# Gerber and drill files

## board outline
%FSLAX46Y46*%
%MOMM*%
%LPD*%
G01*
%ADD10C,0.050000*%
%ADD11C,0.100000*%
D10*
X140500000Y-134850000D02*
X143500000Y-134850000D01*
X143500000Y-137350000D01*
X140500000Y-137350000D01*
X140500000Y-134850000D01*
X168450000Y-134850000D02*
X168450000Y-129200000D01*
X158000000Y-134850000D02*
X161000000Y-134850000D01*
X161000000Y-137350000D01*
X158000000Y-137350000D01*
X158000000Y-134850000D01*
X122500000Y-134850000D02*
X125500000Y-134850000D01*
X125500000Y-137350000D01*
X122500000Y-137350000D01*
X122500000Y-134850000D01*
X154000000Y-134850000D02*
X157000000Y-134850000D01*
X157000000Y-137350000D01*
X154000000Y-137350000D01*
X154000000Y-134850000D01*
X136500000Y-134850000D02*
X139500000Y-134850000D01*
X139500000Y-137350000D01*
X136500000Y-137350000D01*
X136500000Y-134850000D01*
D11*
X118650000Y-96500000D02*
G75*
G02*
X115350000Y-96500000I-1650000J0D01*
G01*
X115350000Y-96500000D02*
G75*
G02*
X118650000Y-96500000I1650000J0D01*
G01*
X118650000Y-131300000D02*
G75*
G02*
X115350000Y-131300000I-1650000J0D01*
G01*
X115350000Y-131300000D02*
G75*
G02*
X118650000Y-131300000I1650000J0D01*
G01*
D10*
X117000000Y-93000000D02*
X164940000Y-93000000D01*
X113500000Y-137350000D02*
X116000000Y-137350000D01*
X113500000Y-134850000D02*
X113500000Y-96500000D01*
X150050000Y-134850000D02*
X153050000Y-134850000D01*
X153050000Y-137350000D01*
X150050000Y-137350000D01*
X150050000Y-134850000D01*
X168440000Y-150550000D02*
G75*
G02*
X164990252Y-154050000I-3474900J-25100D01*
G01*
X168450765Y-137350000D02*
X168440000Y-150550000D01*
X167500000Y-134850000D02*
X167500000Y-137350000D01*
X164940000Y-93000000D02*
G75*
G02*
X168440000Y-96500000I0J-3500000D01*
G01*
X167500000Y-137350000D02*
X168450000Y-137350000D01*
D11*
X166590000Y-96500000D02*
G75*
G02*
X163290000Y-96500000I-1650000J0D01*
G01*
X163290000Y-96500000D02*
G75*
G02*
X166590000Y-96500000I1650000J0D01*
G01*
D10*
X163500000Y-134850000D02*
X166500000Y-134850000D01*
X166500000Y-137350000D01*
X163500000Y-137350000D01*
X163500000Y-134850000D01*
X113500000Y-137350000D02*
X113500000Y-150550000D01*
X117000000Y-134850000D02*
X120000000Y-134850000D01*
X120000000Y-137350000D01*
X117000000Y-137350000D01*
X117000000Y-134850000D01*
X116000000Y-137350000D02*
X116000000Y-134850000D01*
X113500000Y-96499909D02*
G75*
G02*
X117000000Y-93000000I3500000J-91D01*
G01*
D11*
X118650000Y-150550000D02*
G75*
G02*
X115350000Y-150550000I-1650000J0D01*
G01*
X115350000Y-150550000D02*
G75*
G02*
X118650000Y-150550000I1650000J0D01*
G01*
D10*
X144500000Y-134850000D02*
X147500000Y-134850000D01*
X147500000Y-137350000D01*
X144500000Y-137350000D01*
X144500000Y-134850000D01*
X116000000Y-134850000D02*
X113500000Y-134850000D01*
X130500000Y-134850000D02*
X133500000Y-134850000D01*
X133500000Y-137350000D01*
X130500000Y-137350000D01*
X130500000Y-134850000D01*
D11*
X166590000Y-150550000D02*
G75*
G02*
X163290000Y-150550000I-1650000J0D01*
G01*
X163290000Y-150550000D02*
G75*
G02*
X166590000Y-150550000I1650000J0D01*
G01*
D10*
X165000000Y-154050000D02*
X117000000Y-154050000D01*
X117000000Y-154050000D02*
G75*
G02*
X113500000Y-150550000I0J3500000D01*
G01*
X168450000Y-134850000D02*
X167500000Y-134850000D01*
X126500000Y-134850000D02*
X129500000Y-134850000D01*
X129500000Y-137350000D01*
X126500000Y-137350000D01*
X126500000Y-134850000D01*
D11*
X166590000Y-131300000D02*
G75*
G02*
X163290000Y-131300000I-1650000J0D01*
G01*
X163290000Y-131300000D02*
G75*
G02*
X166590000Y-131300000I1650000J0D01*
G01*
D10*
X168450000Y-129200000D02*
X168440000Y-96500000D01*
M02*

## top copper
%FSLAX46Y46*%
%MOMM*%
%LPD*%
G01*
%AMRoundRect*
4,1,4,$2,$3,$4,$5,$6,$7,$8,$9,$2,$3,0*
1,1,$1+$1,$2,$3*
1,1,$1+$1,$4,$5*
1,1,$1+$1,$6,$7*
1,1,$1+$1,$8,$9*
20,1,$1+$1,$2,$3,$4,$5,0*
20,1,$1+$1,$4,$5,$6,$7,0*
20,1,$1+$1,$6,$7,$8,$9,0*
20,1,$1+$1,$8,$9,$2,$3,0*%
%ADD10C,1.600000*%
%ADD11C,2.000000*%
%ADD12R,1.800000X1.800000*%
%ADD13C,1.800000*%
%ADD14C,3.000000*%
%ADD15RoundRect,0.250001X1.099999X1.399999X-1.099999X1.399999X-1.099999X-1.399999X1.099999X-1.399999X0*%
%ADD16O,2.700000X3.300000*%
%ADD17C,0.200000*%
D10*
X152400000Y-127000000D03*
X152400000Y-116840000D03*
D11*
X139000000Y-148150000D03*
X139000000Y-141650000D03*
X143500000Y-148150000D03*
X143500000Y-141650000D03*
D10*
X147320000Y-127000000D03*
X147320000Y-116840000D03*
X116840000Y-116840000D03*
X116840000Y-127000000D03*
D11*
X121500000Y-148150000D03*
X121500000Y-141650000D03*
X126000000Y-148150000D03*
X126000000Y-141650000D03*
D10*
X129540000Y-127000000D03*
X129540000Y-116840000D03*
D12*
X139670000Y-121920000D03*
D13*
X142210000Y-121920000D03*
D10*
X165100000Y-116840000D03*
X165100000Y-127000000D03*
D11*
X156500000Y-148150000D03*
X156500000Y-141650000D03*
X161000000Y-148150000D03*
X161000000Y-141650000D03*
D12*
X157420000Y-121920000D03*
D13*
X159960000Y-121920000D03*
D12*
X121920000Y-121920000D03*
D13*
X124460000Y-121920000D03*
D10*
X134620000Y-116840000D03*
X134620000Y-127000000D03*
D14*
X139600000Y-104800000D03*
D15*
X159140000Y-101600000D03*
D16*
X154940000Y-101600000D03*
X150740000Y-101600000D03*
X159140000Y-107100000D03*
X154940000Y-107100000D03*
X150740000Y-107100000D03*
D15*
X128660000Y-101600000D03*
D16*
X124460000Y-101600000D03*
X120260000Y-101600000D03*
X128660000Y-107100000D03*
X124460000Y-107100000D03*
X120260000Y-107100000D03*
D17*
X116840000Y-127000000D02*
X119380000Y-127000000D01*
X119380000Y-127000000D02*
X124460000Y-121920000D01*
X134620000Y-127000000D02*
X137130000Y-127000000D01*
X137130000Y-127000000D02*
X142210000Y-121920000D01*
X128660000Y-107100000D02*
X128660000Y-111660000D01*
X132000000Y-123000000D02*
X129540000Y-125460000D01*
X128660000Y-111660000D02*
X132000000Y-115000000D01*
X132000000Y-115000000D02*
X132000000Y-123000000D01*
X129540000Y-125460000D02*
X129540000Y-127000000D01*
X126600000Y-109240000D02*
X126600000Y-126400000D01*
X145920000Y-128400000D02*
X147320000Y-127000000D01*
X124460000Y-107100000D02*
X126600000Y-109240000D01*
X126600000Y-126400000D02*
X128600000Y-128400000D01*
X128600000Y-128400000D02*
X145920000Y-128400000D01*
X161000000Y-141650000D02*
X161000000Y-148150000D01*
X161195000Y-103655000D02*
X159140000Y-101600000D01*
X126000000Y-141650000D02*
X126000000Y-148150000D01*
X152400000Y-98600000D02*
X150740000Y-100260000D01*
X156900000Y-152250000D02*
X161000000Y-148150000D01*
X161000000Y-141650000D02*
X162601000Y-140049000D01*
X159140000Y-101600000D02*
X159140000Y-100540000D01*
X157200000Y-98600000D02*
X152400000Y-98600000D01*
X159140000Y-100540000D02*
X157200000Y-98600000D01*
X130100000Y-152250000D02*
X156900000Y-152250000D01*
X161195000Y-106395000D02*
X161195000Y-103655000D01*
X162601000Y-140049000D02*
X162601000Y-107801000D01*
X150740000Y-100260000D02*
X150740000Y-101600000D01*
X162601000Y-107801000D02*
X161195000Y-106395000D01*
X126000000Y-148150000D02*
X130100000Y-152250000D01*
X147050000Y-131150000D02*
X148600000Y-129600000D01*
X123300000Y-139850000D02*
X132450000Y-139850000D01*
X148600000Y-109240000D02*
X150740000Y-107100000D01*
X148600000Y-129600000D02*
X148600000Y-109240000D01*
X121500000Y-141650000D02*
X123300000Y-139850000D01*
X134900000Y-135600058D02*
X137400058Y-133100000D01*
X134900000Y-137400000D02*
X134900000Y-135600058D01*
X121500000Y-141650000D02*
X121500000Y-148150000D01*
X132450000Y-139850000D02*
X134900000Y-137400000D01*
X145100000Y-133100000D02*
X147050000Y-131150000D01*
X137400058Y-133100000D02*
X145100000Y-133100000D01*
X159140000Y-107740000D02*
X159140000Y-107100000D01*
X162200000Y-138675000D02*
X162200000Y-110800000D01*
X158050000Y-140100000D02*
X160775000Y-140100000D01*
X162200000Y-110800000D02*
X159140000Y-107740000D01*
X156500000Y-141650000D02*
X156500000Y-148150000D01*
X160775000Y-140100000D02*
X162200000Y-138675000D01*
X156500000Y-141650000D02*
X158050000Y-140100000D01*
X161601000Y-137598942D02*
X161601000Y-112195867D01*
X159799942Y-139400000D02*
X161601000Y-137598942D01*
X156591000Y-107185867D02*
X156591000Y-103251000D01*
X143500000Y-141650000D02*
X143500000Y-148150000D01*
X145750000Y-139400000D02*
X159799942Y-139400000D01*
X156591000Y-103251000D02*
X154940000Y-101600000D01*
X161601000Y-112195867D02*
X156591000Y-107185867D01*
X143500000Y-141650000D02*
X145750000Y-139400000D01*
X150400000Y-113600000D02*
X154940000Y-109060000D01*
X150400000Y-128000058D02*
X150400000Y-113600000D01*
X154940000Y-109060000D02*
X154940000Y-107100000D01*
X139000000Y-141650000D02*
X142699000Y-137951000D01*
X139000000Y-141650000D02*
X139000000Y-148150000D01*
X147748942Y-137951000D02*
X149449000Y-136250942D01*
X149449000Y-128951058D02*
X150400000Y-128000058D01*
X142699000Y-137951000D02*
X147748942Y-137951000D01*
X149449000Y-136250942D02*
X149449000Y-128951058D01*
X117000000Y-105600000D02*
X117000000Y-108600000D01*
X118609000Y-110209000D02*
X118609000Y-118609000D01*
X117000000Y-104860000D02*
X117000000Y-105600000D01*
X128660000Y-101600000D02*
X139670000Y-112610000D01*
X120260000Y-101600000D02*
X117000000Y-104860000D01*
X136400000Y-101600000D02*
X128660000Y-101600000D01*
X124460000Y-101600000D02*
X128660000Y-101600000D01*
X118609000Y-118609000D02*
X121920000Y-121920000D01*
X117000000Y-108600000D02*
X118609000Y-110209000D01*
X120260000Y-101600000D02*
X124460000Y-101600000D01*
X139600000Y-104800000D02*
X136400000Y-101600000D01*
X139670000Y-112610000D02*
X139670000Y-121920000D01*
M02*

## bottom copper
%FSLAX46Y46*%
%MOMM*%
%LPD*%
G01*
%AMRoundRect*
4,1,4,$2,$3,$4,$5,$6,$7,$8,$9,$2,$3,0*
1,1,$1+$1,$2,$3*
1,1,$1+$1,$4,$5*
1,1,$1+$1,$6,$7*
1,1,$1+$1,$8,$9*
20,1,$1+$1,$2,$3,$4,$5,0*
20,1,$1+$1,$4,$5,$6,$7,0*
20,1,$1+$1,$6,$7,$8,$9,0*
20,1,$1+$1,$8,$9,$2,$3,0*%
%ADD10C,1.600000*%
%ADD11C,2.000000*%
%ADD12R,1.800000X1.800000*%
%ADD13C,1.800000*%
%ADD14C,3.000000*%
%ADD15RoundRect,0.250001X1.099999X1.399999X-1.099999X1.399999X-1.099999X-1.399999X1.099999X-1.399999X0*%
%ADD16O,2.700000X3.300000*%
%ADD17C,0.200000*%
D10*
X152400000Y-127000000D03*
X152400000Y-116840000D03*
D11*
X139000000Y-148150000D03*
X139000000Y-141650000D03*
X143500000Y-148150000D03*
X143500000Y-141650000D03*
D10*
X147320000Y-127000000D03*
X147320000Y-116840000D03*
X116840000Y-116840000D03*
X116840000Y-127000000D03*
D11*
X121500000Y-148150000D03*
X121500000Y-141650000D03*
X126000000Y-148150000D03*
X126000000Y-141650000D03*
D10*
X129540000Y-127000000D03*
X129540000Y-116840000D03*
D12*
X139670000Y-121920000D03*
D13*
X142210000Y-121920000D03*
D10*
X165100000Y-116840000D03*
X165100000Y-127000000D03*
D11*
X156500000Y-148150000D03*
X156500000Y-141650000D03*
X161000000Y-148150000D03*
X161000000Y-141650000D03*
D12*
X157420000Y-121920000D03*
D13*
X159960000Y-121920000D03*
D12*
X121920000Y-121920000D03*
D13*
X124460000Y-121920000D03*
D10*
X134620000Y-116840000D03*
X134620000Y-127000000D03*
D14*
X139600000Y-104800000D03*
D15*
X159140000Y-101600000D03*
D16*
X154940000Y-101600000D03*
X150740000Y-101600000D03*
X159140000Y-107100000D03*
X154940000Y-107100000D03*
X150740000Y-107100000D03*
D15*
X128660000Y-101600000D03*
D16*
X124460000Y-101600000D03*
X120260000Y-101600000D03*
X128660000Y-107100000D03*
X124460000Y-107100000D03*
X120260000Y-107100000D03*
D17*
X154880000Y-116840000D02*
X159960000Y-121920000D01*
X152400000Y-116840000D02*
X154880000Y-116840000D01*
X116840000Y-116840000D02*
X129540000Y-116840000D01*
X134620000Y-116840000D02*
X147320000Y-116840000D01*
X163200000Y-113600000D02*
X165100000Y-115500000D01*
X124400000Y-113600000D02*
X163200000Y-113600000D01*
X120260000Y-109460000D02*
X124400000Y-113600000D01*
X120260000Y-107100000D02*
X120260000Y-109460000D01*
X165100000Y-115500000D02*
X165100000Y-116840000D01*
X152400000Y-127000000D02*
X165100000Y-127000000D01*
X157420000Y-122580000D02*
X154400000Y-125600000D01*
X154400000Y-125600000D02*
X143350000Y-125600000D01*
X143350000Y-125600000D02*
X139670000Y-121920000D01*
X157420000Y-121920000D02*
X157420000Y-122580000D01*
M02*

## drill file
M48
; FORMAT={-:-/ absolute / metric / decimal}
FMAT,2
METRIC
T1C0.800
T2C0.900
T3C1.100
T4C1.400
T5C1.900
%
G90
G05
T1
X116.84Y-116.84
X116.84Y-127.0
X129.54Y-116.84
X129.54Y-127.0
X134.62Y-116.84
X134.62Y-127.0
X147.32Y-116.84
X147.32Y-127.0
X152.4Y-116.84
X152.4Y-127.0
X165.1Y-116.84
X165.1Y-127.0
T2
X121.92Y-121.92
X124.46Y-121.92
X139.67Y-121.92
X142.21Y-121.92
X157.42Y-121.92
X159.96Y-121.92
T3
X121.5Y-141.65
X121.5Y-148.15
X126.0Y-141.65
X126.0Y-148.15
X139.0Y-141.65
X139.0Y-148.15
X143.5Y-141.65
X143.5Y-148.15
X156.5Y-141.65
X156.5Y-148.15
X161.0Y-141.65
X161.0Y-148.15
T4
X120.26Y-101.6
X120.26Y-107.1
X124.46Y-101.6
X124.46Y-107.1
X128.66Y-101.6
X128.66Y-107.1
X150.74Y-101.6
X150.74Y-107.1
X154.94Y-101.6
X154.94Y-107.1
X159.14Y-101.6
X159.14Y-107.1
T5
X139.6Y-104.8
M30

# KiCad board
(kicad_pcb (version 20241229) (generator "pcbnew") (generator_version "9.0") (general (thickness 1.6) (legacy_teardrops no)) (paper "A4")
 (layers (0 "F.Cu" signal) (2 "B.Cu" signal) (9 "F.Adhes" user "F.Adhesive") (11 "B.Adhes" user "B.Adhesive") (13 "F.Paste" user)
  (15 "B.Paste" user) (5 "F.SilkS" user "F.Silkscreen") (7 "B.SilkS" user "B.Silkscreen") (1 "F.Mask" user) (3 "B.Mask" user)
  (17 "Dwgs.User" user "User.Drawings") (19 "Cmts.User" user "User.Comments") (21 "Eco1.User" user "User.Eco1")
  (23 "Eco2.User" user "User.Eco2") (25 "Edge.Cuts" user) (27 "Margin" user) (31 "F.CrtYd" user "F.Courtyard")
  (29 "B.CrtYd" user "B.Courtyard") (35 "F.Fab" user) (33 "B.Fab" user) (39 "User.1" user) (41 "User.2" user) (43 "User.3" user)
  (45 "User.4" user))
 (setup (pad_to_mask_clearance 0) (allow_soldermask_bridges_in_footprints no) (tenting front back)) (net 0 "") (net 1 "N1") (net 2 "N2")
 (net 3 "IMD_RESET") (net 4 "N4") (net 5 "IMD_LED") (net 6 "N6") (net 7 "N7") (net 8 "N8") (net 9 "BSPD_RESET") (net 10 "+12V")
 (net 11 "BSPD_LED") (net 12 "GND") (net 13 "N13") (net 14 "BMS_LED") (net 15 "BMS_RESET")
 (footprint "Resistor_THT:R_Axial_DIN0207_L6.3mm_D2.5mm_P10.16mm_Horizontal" (layer "F.Cu") (at 152.4 127 90)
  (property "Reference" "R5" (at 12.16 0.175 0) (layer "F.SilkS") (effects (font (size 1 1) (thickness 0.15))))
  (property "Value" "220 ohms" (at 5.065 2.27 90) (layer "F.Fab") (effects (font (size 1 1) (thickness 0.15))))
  (pad "1" thru_hole circle (at 0 0 90) (size 1.6 1.6) (drill 0.8) (layers "*.Cu" "*.Mask") (remove_unused_layers no) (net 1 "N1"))
  (pad "2" thru_hole circle (at 10.16 0 90) (size 1.6 1.6) (drill 0.8) (layers "*.Cu" "*.Mask") (remove_unused_layers no) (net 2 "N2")))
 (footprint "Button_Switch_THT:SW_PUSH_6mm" (layer "F.Cu") (at 139 148.15 90)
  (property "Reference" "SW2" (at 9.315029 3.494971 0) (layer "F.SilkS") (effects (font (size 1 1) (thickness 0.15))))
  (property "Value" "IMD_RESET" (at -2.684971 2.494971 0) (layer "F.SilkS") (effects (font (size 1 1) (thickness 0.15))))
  (pad "1" thru_hole circle (at 0 0 180) (size 2 2) (drill 1.1) (layers "*.Cu" "*.Mask") (remove_unused_layers no) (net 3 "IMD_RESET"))
  (pad "1" thru_hole circle (at 6.5 0 180) (size 2 2) (drill 1.1) (layers "*.Cu" "*.Mask") (remove_unused_layers no) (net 3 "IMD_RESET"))
  (pad "2" thru_hole circle (at 0 4.5 180) (size 2 2) (drill 1.1) (layers "*.Cu" "*.Mask") (remove_unused_layers no) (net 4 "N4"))
  (pad "2" thru_hole circle (at 6.5 4.5 180) (size 2 2) (drill 1.1) (layers "*.Cu" "*.Mask") (remove_unused_layers no) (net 4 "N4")))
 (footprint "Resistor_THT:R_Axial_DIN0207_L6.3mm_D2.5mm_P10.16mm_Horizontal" (layer "F.Cu") (at 147.32 127 90)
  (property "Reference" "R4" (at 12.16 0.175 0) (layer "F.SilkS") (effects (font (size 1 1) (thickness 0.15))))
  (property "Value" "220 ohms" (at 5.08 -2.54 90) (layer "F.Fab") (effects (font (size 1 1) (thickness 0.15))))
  (pad "1" thru_hole circle (at 0 0 90) (size 1.6 1.6) (drill 0.8) (layers "*.Cu" "*.Mask") (remove_unused_layers no) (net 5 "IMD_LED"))
  (pad "2" thru_hole circle (at 10.16 0 90) (size 1.6 1.6) (drill 0.8) (layers "*.Cu" "*.Mask") (remove_unused_layers no) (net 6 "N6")))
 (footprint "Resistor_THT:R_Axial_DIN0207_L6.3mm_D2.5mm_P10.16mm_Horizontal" (layer "F.Cu") (at 116.84 116.84 -90)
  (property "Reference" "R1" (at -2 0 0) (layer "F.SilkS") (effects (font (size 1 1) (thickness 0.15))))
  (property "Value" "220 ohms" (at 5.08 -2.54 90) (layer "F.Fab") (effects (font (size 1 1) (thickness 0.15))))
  (pad "1" thru_hole circle (at 0 0 270) (size 1.6 1.6) (drill 0.8) (layers "*.Cu" "*.Mask") (remove_unused_layers no) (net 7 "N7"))
  (pad "2" thru_hole circle (at 10.16 0 270) (size 1.6 1.6) (drill 0.8) (layers "*.Cu" "*.Mask") (remove_unused_layers no) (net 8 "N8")))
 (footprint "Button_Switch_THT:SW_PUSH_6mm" (layer "F.Cu") (at 121.5 148.15 90)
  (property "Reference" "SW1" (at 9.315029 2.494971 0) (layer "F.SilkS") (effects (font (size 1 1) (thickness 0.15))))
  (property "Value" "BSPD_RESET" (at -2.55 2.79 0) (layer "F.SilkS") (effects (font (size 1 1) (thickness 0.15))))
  (pad "1" thru_hole circle (at 0 0 180) (size 2 2) (drill 1.1) (layers "*.Cu" "*.Mask") (remove_unused_layers no) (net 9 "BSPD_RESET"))
  (pad "1" thru_hole circle (at 6.5 0 180) (size 2 2) (drill 1.1) (layers "*.Cu" "*.Mask") (remove_unused_layers no) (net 9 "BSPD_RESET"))
  (pad "2" thru_hole circle (at 0 4.5 180) (size 2 2) (drill 1.1) (layers "*.Cu" "*.Mask") (remove_unused_layers no) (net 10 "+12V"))
  (pad "2" thru_hole circle (at 6.5 4.5 180) (size 2 2) (drill 1.1) (layers "*.Cu" "*.Mask") (remove_unused_layers no) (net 10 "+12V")))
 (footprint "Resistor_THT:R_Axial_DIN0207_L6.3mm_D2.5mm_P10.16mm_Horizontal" (layer "F.Cu") (at 129.54 127 90)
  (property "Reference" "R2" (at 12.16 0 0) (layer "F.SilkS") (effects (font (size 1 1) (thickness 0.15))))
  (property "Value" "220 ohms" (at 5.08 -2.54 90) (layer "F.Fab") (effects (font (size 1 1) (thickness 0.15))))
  (pad "1" thru_hole circle (at 0 0 90) (size 1.6 1.6) (drill 0.8) (layers "*.Cu" "*.Mask") (remove_unused_layers no) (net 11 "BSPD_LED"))
  (pad "2" thru_hole circle (at 10.16 0 90) (size 1.6 1.6) (drill 0.8) (layers "*.Cu" "*.Mask") (remove_unused_layers no) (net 7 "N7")))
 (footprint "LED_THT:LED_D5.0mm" (layer "F.Cu") (at 139.67 121.92)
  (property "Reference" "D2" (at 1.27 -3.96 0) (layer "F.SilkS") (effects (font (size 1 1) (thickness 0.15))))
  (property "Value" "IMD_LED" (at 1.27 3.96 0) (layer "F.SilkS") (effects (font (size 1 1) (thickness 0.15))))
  (pad "1" thru_hole rect (at 0 0) (size 1.8 1.8) (drill 0.9) (layers "*.Cu" "*.Mask") (remove_unused_layers no) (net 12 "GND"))
  (pad "2" thru_hole circle (at 2.54 0) (size 1.8 1.8) (drill 0.9) (layers "*.Cu" "*.Mask") (remove_unused_layers no) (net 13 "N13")))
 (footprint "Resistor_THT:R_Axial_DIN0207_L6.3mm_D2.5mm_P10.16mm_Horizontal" (layer "F.Cu") (at 165.1 116.84 -90)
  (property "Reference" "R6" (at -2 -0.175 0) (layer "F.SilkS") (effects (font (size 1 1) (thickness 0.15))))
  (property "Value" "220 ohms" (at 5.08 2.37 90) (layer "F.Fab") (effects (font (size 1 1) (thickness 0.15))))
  (pad "1" thru_hole circle (at 0 0 270) (size 1.6 1.6) (drill 0.8) (layers "*.Cu" "*.Mask") (remove_unused_layers no) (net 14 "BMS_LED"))
  (pad "2" thru_hole circle (at 10.16 0 270) (size 1.6 1.6) (drill 0.8) (layers "*.Cu" "*.Mask") (remove_unused_layers no) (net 1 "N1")))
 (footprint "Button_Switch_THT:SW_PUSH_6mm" (layer "F.Cu") (at 156.5 148.15 90)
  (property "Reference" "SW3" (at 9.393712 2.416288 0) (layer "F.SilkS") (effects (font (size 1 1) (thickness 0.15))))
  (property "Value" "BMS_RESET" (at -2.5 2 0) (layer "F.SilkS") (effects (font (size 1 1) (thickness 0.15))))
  (pad "1" thru_hole circle (at 0 0 180) (size 2 2) (drill 1.1) (layers "*.Cu" "*.Mask") (remove_unused_layers no) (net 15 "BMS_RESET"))
  (pad "1" thru_hole circle (at 6.5 0 180) (size 2 2) (drill 1.1) (layers "*.Cu" "*.Mask") (remove_unused_layers no) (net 15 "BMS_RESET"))
  (pad "2" thru_hole circle (at 0 4.5 180) (size 2 2) (drill 1.1) (layers "*.Cu" "*.Mask") (remove_unused_layers no) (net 10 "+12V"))
  (pad "2" thru_hole circle (at 6.5 4.5 180) (size 2 2) (drill 1.1) (layers "*.Cu" "*.Mask") (remove_unused_layers no) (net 10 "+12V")))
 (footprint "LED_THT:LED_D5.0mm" (layer "F.Cu") (at 157.42 121.92)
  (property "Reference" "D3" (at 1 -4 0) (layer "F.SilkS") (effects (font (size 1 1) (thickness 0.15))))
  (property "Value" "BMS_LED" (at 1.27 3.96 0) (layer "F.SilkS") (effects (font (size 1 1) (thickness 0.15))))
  (pad "1" thru_hole rect (at 0 0) (size 1.8 1.8) (drill 0.9) (layers "*.Cu" "*.Mask") (remove_unused_layers no) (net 12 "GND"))
  (pad "2" thru_hole circle (at 2.54 0) (size 1.8 1.8) (drill 0.9) (layers "*.Cu" "*.Mask") (remove_unused_layers no) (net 2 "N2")))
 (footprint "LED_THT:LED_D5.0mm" (layer "F.Cu") (at 121.92 121.92)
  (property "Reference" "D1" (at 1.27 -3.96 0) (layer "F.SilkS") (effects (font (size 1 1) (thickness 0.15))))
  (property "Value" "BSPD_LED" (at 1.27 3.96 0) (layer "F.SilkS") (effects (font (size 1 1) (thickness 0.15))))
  (pad "1" thru_hole rect (at 0 0) (size 1.8 1.8) (drill 0.9) (layers "*.Cu" "*.Mask") (remove_unused_layers no) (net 12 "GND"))
  (pad "2" thru_hole circle (at 2.54 0) (size 1.8 1.8) (drill 0.9) (layers "*.Cu" "*.Mask") (remove_unused_layers no) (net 8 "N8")))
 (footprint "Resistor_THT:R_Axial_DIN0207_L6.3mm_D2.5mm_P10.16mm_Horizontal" (layer "F.Cu") (at 134.62 116.84 -90)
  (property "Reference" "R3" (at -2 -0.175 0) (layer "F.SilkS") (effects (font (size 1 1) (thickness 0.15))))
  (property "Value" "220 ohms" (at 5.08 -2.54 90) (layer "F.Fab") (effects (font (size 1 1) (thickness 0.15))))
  (pad "1" thru_hole circle (at 0 0 270) (size 1.6 1.6) (drill 0.8) (layers "*.Cu" "*.Mask") (remove_unused_layers no) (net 6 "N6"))
  (pad "2" thru_hole circle (at 10.16 0 270) (size 1.6 1.6) (drill 0.8) (layers "*.Cu" "*.Mask") (remove_unused_layers no) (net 13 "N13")))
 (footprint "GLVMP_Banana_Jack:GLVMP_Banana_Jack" (layer "B.Cu") (at 139.6 104.8 180)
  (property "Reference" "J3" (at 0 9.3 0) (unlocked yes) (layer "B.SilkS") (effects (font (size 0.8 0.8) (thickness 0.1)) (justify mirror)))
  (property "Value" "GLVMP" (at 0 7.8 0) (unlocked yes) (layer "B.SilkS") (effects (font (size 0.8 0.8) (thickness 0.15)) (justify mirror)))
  (pad "1" thru_hole circle (at 0 0 180) (size 3 3) (drill 1.9) (layers "*.Cu" "*.Mask") (remove_unused_layers no) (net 12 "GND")))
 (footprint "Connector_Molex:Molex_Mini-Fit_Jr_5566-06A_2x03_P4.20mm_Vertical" (layer "B.Cu") (at 159.14 101.6 180)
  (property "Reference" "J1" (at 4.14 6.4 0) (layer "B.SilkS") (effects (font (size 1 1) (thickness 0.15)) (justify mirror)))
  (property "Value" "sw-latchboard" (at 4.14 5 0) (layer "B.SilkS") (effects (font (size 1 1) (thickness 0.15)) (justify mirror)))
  (pad "1" thru_hole roundrect (at 0 0 180) (size 2.7 3.3) (drill 1.4) (layers "*.Cu" "*.Mask") (remove_unused_layers no)
   (roundrect_rratio 0.092593) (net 10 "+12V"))
  (pad "2" thru_hole oval (at 4.2 0 180) (size 2.7 3.3) (drill 1.4) (layers "*.Cu" "*.Mask") (remove_unused_layers no) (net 4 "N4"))
  (pad "3" thru_hole oval (at 8.4 0 180) (size 2.7 3.3) (drill 1.4) (layers "*.Cu" "*.Mask") (remove_unused_layers no) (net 10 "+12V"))
  (pad "4" thru_hole oval (at 0 -5.5 180) (size 2.7 3.3) (drill 1.4) (layers "*.Cu" "*.Mask") (remove_unused_layers no) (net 15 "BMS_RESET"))
  (pad "5" thru_hole oval (at 4.2 -5.5 180) (size 2.7 3.3) (drill 1.4) (layers "*.Cu" "*.Mask") (remove_unused_layers no)
   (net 3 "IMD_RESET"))
  (pad "6" thru_hole oval (at 8.4 -5.5 180) (size 2.7 3.3) (drill 1.4) (layers "*.Cu" "*.Mask") (remove_unused_layers no)
   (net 9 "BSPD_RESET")))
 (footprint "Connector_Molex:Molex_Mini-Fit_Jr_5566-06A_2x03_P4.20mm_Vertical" (layer "B.Cu") (at 128.66 101.6 180)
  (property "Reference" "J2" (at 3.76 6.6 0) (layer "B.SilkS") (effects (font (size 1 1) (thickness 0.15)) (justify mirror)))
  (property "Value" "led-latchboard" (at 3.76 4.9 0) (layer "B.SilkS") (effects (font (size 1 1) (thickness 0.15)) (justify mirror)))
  (pad "1" thru_hole roundrect (at 0 0 180) (size 2.7 3.3) (drill 1.4) (layers "*.Cu" "*.Mask") (remove_unused_layers no)
   (roundrect_rratio 0.092593) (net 12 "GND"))
  (pad "2" thru_hole oval (at 4.2 0 180) (size 2.7 3.3) (drill 1.4) (layers "*.Cu" "*.Mask") (remove_unused_layers no) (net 12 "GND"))
  (pad "3" thru_hole oval (at 8.4 0 180) (size 2.7 3.3) (drill 1.4) (layers "*.Cu" "*.Mask") (remove_unused_layers no) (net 12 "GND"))
  (pad "4" thru_hole oval (at 0 -5.5 180) (size 2.7 3.3) (drill 1.4) (layers "*.Cu" "*.Mask") (remove_unused_layers no) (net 11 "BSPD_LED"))
  (pad "5" thru_hole oval (at 4.2 -5.5 180) (size 2.7 3.3) (drill 1.4) (layers "*.Cu" "*.Mask") (remove_unused_layers no) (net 5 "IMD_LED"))
  (pad "6" thru_hole oval (at 8.4 -5.5 180) (size 2.7 3.3) (drill 1.4) (layers "*.Cu" "*.Mask") (remove_unused_layers no) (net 14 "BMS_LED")))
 (gr_rect (start 140.5 134.85) (end 143.5 137.35) (stroke (width 0.05) (type default)) (fill no) (layer "Edge.Cuts"))
 (gr_line (start 168.45 134.85) (end 168.45 129.2) (stroke (width 0.05) (type default)) (layer "Edge.Cuts"))
 (gr_rect (start 158 134.85) (end 161 137.35) (stroke (width 0.05) (type default)) (fill no) (layer "Edge.Cuts"))
 (gr_rect (start 122.5 134.85) (end 125.5 137.35) (stroke (width 0.05) (type default)) (fill no) (layer "Edge.Cuts"))
 (gr_rect (start 154 134.85) (end 157 137.35) (stroke (width 0.05) (type default)) (fill no) (layer "Edge.Cuts"))
 (gr_rect (start 136.5 134.85) (end 139.5 137.35) (stroke (width 0.05) (type default)) (fill no) (layer "Edge.Cuts"))
 (gr_circle (center 117 96.5) (end 118.65 96.5) (stroke (width 0.1) (type solid)) (fill no) (layer "Edge.Cuts"))
 (gr_circle (center 117 131.3) (end 115.35 131.3) (stroke (width 0.1) (type solid)) (fill no) (layer "Edge.Cuts"))
 (gr_line (start 117 93) (end 164.94 93) (stroke (width 0.05) (type default)) (layer "Edge.Cuts"))
 (gr_line (start 113.5 137.35) (end 116 137.35) (stroke (width 0.05) (type default)) (layer "Edge.Cuts"))
 (gr_line (start 113.5 134.85) (end 113.5 96.5) (stroke (width 0.05) (type default)) (layer "Edge.Cuts"))
 (gr_rect (start 150.05 134.85) (end 153.05 137.35) (stroke (width 0.05) (type default)) (fill no) (layer "Edge.Cuts"))
 (gr_arc (start 168.44 150.55) (mid 167.44 153.014466) (end 164.990252 154.05) (stroke (width 0.05) (type solid)) (layer "Edge.Cuts"))
 (gr_line (start 168.450765 137.35) (end 168.44 150.55) (stroke (width 0.05) (type default)) (layer "Edge.Cuts"))
 (gr_line (start 167.5 134.85) (end 167.5 137.35) (stroke (width 0.05) (type default)) (layer "Edge.Cuts"))
 (gr_arc (start 164.94 93) (mid 167.414874 94.025126) (end 168.44 96.5) (stroke (width 0.05) (type solid)) (layer "Edge.Cuts"))
 (gr_line (start 167.5 137.35) (end 168.45 137.35) (stroke (width 0.05) (type default)) (layer "Edge.Cuts"))
 (gr_circle (center 164.94 96.5) (end 166.59 96.5) (stroke (width 0.1) (type solid)) (fill no) (layer "Edge.Cuts"))
 (gr_rect (start 163.5 134.85) (end 166.5 137.35) (stroke (width 0.05) (type default)) (fill no) (layer "Edge.Cuts"))
 (gr_line (start 113.5 137.35) (end 113.5 150.55) (stroke (width 0.05) (type solid)) (layer "Edge.Cuts"))
 (gr_rect (start 117 134.85) (end 120 137.35) (stroke (width 0.05) (type default)) (fill no) (layer "Edge.Cuts"))
 (gr_line (start 116 137.35) (end 116 134.85) (stroke (width 0.05) (type default)) (layer "Edge.Cuts"))
 (gr_arc (start 113.5 96.499909) (mid 114.525158 94.025094) (end 117 93) (stroke (width 0.05) (type default)) (layer "Edge.Cuts"))
 (gr_circle (center 117 150.55) (end 115.35 150.55) (stroke (width 0.1) (type solid)) (fill no) (layer "Edge.Cuts"))
 (gr_rect (start 144.5 134.85) (end 147.5 137.35) (stroke (width 0.05) (type default)) (fill no) (layer "Edge.Cuts"))
 (gr_line (start 116 134.85) (end 113.5 134.85) (stroke (width 0.05) (type default)) (layer "Edge.Cuts"))
 (gr_rect (start 130.5 134.85) (end 133.5 137.35) (stroke (width 0.05) (type default)) (fill no) (layer "Edge.Cuts"))
 (gr_circle (center 164.94 150.55) (end 163.29 150.55) (stroke (width 0.1) (type solid)) (fill no) (layer "Edge.Cuts"))
 (gr_line (start 165 154.05) (end 117 154.05) (stroke (width 0.05) (type solid)) (layer "Edge.Cuts"))
 (gr_arc (start 117 154.05) (mid 114.525126 153.024874) (end 113.5 150.55) (stroke (width 0.05) (type solid)) (layer "Edge.Cuts"))
 (gr_line (start 168.45 134.85) (end 167.5 134.85) (stroke (width 0.05) (type default)) (layer "Edge.Cuts"))
 (gr_rect (start 126.5 134.85) (end 129.5 137.35) (stroke (width 0.05) (type default)) (fill no) (layer "Edge.Cuts"))
 (gr_circle (center 164.94 131.3) (end 166.59 131.3) (stroke (width 0.1) (type solid)) (fill no) (layer "Edge.Cuts"))
 (gr_line (start 168.45 129.2) (end 168.44 96.5) (stroke (width 0.05) (type default)) (layer "Edge.Cuts"))
 (segment (start 116.84 127) (end 119.38 127) (width 0.2) (layer "F.Cu") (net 8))
 (segment (start 119.38 127) (end 124.46 121.92) (width 0.2) (layer "F.Cu") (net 8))
 (segment (start 134.62 127) (end 137.13 127) (width 0.2) (layer "F.Cu") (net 13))
 (segment (start 137.13 127) (end 142.21 121.92) (width 0.2) (layer "F.Cu") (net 13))
 (segment (start 154.88 116.84) (end 159.96 121.92) (width 0.2) (layer "B.Cu") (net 2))
 (segment (start 152.4 116.84) (end 154.88 116.84) (width 0.2) (layer "B.Cu") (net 2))
 (segment (start 116.84 116.84) (end 129.54 116.84) (width 0.2) (layer "B.Cu") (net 7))
 (segment (start 128.66 107.1) (end 128.66 111.66) (width 0.2) (layer "F.Cu") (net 11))
 (segment (start 132 123) (end 129.54 125.46) (width 0.2) (layer "F.Cu") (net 11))
 (segment (start 128.66 111.66) (end 132 115) (width 0.2) (layer "F.Cu") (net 11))
 (segment (start 132 115) (end 132 123) (width 0.2) (layer "F.Cu") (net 11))
 (segment (start 129.54 125.46) (end 129.54 127) (width 0.2) (layer "F.Cu") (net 11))
 (segment (start 134.62 116.84) (end 147.32 116.84) (width 0.2) (layer "B.Cu") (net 6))
 (segment (start 126.6 109.24) (end 126.6 126.4) (width 0.2) (layer "F.Cu") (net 5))
 (segment (start 145.92 128.4) (end 147.32 127) (width 0.2) (layer "F.Cu") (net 5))
 (segment (start 124.46 107.1) (end 126.6 109.24) (width 0.2) (layer "F.Cu") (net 5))
 (segment (start 126.6 126.4) (end 128.6 128.4) (width 0.2) (layer "F.Cu") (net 5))
 (segment (start 128.6 128.4) (end 145.92 128.4) (width 0.2) (layer "F.Cu") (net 5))
 (segment (start 163.2 113.6) (end 165.1 115.5) (width 0.2) (layer "B.Cu") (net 14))
 (segment (start 124.4 113.6) (end 163.2 113.6) (width 0.2) (layer "B.Cu") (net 14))
 (segment (start 120.26 109.46) (end 124.4 113.6) (width 0.2) (layer "B.Cu") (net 14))
 (segment (start 120.26 107.1) (end 120.26 109.46) (width 0.2) (layer "B.Cu") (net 14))
 (segment (start 165.1 115.5) (end 165.1 116.84) (width 0.2) (layer "B.Cu") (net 14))
 (segment (start 161 141.65) (end 161 148.15) (width 0.2) (layer "F.Cu") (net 10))
 (segment (start 161.195 103.655) (end 159.14 101.6) (width 0.2) (layer "F.Cu") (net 10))
 (segment (start 126 141.65) (end 126 148.15) (width 0.2) (layer "F.Cu") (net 10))
 (segment (start 152.4 98.6) (end 150.74 100.26) (width 0.2) (layer "F.Cu") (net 10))
 (segment (start 156.9 152.25) (end 161 148.15) (width 0.2) (layer "F.Cu") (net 10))
 (segment (start 161 141.65) (end 162.601 140.049) (width 0.2) (layer "F.Cu") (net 10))
 (segment (start 159.14 101.6) (end 159.14 100.54) (width 0.2) (layer "F.Cu") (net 10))
 (segment (start 157.2 98.6) (end 152.4 98.6) (width 0.2) (layer "F.Cu") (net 10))
 (segment (start 159.14 100.54) (end 157.2 98.6) (width 0.2) (layer "F.Cu") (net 10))
 (segment (start 130.1 152.25) (end 156.9 152.25) (width 0.2) (layer "F.Cu") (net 10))
 (segment (start 161.195 106.395) (end 161.195 103.655) (width 0.2) (layer "F.Cu") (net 10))
 (segment (start 162.601 140.049) (end 162.601 107.801) (width 0.2) (layer "F.Cu") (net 10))
 (segment (start 150.74 100.26) (end 150.74 101.6) (width 0.2) (layer "F.Cu") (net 10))
 (segment (start 162.601 107.801) (end 161.195 106.395) (width 0.2) (layer "F.Cu") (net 10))
 (segment (start 126 148.15) (end 130.1 152.25) (width 0.2) (layer "F.Cu") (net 10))
 (segment (start 147.05 131.15) (end 148.6 129.6) (width 0.2) (layer "F.Cu") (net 9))
 (segment (start 123.3 139.85) (end 132.45 139.85) (width 0.2) (layer "F.Cu") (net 9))
 (segment (start 148.6 109.24) (end 150.74 107.1) (width 0.2) (layer "F.Cu") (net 9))
 (segment (start 148.6 129.6) (end 148.6 109.24) (width 0.2) (layer "F.Cu") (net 9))
 (segment (start 121.5 141.65) (end 123.3 139.85) (width 0.2) (layer "F.Cu") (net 9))
 (segment (start 134.9 135.600058) (end 137.400058 133.1) (width 0.2) (layer "F.Cu") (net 9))
 (segment (start 134.9 137.4) (end 134.9 135.600058) (width 0.2) (layer "F.Cu") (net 9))
 (segment (start 121.5 141.65) (end 121.5 148.15) (width 0.2) (layer "F.Cu") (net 9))
 (segment (start 132.45 139.85) (end 134.9 137.4) (width 0.2) (layer "F.Cu") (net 9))
 (segment (start 145.1 133.1) (end 147.05 131.15) (width 0.2) (layer "F.Cu") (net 9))
 (segment (start 137.400058 133.1) (end 145.1 133.1) (width 0.2) (layer "F.Cu") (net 9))
 (segment (start 159.14 107.74) (end 159.14 107.1) (width 0.2) (layer "F.Cu") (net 15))
 (segment (start 162.2 138.675) (end 162.2 110.8) (width 0.2) (layer "F.Cu") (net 15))
 (segment (start 158.05 140.1) (end 160.775 140.1) (width 0.2) (layer "F.Cu") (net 15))
 (segment (start 162.2 110.8) (end 159.14 107.74) (width 0.2) (layer "F.Cu") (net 15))
 (segment (start 156.5 141.65) (end 156.5 148.15) (width 0.2) (layer "F.Cu") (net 15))
 (segment (start 160.775 140.1) (end 162.2 138.675) (width 0.2) (layer "F.Cu") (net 15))
 (segment (start 156.5 141.65) (end 158.05 140.1) (width 0.2) (layer "F.Cu") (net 15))
 (segment (start 161.601 137.598942) (end 161.601 112.195867) (width 0.2) (layer "F.Cu") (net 4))
 (segment (start 159.799942 139.4) (end 161.601 137.598942) (width 0.2) (layer "F.Cu") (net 4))
 (segment (start 156.591 107.185867) (end 156.591 103.251) (width 0.2) (layer "F.Cu") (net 4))
 (segment (start 143.5 141.65) (end 143.5 148.15) (width 0.2) (layer "F.Cu") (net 4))
 (segment (start 145.75 139.4) (end 159.799942 139.4) (width 0.2) (layer "F.Cu") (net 4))
 (segment (start 156.591 103.251) (end 154.94 101.6) (width 0.2) (layer "F.Cu") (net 4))
 (segment (start 161.601 112.195867) (end 156.591 107.185867) (width 0.2) (layer "F.Cu") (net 4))
 (segment (start 143.5 141.65) (end 145.75 139.4) (width 0.2) (layer "F.Cu") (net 4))
 (segment (start 150.4 113.6) (end 154.94 109.06) (width 0.2) (layer "F.Cu") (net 3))
 (segment (start 150.4 128.000058) (end 150.4 113.6) (width 0.2) (layer "F.Cu") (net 3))
 (segment (start 154.94 109.06) (end 154.94 107.1) (width 0.2) (layer "F.Cu") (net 3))
 (segment (start 139 141.65) (end 142.699 137.951) (width 0.2) (layer "F.Cu") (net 3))
 (segment (start 139 141.65) (end 139 148.15) (width 0.2) (layer "F.Cu") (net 3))
 (segment (start 147.748942 137.951) (end 149.449 136.250942) (width 0.2) (layer "F.Cu") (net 3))
 (segment (start 149.449 128.951058) (end 150.4 128.000058) (width 0.2) (layer "F.Cu") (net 3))
 (segment (start 142.699 137.951) (end 147.748942 137.951) (width 0.2) (layer "F.Cu") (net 3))
 (segment (start 149.449 136.250942) (end 149.449 128.951058) (width 0.2) (layer "F.Cu") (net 3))
 (segment (start 152.4 127) (end 165.1 127) (width 0.2) (layer "B.Cu") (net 1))
 (segment (start 117 105.6) (end 117 108.6) (width 0.2) (layer "F.Cu") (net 12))
 (segment (start 118.609 110.209) (end 118.609 118.609) (width 0.2) (layer "F.Cu") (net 12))
 (segment (start 117 104.86) (end 117 105.6) (width 0.2) (layer "F.Cu") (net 12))
 (segment (start 128.66 101.6) (end 139.67 112.61) (width 0.2) (layer "F.Cu") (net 12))
 (segment (start 120.26 101.6) (end 117 104.86) (width 0.2) (layer "F.Cu") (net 12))
 (segment (start 136.4 101.6) (end 128.66 101.6) (width 0.2) (layer "F.Cu") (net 12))
 (segment (start 124.46 101.6) (end 128.66 101.6) (width 0.2) (layer "F.Cu") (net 12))
 (segment (start 118.609 118.609) (end 121.92 121.92) (width 0.2) (layer "F.Cu") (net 12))
 (segment (start 117 108.6) (end 118.609 110.209) (width 0.2) (layer "F.Cu") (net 12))
 (segment (start 120.26 101.6) (end 124.46 101.6) (width 0.2) (layer "F.Cu") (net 12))
 (segment (start 139.6 104.8) (end 136.4 101.6) (width 0.2) (layer "F.Cu") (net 12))
 (segment (start 139.67 112.61) (end 139.67 121.92) (width 0.2) (layer "F.Cu") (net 12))
 (segment (start 157.42 122.58) (end 154.4 125.6) (width 0.2) (layer "B.Cu") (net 12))
 (segment (start 154.4 125.6) (end 143.35 125.6) (width 0.2) (layer "B.Cu") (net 12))
 (segment (start 143.35 125.6) (end 139.67 121.92) (width 0.2) (layer "B.Cu") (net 12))
 (segment (start 157.42 121.92) (end 157.42 122.58) (width 0.2) (layer "B.Cu") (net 12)))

